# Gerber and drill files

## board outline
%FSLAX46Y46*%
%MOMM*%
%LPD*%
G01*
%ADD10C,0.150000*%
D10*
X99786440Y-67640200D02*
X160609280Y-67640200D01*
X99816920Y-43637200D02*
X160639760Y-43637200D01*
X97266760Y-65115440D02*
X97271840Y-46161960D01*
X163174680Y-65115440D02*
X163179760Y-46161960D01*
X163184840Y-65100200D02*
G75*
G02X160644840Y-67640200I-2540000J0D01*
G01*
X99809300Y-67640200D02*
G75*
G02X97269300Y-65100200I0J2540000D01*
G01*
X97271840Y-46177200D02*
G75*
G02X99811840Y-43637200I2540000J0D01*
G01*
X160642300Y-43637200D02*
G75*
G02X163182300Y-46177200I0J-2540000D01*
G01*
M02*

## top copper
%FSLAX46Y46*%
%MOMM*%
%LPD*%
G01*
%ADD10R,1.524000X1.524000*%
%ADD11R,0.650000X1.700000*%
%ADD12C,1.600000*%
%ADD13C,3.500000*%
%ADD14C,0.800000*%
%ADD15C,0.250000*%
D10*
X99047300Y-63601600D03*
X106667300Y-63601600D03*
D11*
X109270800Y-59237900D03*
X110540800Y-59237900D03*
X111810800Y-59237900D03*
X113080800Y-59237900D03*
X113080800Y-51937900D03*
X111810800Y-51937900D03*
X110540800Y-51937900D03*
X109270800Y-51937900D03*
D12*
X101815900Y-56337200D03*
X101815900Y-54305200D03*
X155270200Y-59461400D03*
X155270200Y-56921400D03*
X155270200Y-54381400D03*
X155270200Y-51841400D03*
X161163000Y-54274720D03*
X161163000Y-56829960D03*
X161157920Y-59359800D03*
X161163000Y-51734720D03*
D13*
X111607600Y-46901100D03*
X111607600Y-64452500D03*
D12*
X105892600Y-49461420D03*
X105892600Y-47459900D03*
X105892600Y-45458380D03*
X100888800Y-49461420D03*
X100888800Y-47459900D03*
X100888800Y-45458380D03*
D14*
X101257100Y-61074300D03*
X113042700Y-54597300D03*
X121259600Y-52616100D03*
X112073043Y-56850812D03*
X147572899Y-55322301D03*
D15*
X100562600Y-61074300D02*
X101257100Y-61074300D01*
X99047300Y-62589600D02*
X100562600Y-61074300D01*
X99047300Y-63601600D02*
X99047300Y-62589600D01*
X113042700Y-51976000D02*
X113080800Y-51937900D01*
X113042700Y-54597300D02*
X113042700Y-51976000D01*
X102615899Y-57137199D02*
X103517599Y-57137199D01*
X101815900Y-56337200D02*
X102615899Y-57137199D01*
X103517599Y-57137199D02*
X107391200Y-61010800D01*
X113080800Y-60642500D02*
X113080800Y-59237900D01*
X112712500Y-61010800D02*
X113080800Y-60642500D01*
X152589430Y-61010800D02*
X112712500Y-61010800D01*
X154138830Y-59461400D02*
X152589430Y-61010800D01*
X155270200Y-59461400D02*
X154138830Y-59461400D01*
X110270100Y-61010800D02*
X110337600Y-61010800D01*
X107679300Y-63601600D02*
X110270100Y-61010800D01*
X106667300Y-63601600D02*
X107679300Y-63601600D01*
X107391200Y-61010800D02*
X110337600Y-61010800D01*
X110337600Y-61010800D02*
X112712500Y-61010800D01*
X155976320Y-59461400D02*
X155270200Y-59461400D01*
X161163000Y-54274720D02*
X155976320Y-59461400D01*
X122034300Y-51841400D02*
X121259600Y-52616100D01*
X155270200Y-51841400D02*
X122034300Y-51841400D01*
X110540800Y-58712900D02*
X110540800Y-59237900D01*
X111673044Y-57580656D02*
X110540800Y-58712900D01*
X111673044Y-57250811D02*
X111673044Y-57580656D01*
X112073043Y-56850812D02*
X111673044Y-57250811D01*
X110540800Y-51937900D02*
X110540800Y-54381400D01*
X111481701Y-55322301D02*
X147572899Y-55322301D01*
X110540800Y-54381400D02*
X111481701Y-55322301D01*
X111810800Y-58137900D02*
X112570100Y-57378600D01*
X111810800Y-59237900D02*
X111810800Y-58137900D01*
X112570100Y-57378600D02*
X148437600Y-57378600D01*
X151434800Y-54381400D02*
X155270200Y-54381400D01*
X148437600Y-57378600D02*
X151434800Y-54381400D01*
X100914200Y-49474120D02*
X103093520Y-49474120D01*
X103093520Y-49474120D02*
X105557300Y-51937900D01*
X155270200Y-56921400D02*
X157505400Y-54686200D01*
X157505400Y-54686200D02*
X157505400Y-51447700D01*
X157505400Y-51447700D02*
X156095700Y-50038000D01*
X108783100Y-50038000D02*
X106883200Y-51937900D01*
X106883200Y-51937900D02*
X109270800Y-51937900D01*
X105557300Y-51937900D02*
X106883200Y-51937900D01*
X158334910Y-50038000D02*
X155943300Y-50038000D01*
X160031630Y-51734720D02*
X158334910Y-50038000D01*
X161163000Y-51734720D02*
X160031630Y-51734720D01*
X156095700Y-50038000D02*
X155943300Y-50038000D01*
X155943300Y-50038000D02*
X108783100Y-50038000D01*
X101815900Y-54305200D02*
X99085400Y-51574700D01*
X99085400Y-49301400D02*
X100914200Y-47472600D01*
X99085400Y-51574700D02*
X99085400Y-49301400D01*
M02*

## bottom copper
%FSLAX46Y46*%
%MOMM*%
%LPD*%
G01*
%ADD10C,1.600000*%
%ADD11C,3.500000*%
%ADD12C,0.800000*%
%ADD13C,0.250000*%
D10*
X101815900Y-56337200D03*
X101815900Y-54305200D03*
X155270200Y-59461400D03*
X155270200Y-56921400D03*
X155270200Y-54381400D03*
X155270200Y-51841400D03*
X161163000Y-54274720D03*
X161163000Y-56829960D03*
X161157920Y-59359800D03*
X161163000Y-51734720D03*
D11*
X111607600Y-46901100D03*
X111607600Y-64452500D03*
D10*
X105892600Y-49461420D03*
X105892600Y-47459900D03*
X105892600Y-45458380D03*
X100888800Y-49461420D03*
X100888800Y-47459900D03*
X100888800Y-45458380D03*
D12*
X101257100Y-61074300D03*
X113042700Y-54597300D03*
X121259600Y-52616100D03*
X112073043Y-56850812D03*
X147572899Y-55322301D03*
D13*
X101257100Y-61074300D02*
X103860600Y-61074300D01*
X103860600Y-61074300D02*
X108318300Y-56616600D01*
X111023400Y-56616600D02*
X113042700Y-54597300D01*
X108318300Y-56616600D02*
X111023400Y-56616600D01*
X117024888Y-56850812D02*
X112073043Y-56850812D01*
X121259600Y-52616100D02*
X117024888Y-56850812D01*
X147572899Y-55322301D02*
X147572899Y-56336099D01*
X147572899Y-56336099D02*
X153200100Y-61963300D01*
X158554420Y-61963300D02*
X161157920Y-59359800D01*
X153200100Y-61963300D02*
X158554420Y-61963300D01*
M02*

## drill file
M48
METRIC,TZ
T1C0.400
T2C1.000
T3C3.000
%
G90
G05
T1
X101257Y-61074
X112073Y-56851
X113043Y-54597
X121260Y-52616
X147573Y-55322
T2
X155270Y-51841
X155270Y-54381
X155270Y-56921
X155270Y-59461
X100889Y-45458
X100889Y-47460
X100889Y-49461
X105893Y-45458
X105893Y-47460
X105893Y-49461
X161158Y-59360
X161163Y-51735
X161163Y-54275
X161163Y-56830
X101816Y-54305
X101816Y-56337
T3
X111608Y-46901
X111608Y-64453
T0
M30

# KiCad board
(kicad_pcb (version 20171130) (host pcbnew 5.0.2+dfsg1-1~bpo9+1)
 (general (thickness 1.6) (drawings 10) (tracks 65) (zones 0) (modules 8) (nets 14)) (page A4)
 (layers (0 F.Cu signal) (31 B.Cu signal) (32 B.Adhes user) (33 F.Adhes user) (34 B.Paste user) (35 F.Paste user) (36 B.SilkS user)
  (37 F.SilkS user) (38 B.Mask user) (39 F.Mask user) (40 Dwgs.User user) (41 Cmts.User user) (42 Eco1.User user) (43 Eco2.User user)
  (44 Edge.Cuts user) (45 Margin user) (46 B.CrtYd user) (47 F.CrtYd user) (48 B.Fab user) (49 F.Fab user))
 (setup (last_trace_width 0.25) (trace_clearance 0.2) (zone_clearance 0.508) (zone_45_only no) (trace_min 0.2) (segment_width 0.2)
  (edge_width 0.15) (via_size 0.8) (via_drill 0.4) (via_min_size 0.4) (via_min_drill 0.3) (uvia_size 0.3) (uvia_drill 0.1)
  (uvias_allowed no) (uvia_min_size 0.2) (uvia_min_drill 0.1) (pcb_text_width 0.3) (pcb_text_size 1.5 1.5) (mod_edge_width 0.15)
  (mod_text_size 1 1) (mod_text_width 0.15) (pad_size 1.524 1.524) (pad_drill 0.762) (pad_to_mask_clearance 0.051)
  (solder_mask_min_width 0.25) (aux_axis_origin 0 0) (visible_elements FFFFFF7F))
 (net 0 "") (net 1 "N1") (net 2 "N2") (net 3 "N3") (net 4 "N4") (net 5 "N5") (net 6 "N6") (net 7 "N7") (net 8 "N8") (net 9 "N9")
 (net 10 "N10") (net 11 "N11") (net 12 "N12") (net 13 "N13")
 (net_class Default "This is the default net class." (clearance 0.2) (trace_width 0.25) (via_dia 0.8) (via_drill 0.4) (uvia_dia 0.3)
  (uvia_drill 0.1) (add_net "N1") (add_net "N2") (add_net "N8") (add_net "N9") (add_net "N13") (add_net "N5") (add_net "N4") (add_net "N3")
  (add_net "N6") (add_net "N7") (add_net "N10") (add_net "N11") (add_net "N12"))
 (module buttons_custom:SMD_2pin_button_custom (layer F.Cu) (at 102.8573 63.6016 180)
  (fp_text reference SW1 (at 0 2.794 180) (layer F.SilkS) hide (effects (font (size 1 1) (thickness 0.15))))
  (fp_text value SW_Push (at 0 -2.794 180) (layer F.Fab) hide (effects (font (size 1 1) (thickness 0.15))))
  (pad 1 smd rect (at 3.81 0 180) (size 1.524 1.524) (layers F.Cu F.Paste F.Mask) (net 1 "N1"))
  (pad 2 smd rect (at -3.81 0 180) (size 1.524 1.524) (layers F.Cu F.Paste F.Mask) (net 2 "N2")))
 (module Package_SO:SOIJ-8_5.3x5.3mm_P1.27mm (layer F.Cu) (at 111.1758 55.5879 90)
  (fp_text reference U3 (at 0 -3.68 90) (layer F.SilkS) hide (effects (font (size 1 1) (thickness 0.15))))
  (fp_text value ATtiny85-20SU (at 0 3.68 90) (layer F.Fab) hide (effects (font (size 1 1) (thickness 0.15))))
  (pad 1 smd rect (at -3.65 -1.905 90) (size 1.7 0.65) (layers F.Cu F.Paste F.Mask) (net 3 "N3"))
  (pad 2 smd rect (at -3.65 -0.635 90) (size 1.7 0.65) (layers F.Cu F.Paste F.Mask) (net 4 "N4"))
  (pad 3 smd rect (at -3.65 0.635 90) (size 1.7 0.65) (layers F.Cu F.Paste F.Mask) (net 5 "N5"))
  (pad 4 smd rect (at -3.65 1.905 90) (size 1.7 0.65) (layers F.Cu F.Paste F.Mask) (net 2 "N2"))
  (pad 5 smd rect (at 3.65 1.905 90) (size 1.7 0.65) (layers F.Cu F.Paste F.Mask) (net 1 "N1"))
  (pad 6 smd rect (at 3.65 0.635 90) (size 1.7 0.65) (layers F.Cu F.Paste F.Mask) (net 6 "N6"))
  (pad 7 smd rect (at 3.65 -0.635 90) (size 1.7 0.65) (layers F.Cu F.Paste F.Mask) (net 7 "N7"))
  (pad 8 smd rect (at 3.65 -1.905 90) (size 1.7 0.65) (layers F.Cu F.Paste F.Mask) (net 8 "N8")))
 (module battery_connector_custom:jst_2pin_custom (layer F.Cu) (at 101.8159 55.3212 90)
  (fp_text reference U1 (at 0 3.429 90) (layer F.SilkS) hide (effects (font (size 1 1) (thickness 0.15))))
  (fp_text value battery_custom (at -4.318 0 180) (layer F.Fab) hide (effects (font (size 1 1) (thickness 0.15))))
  (pad 1 thru_hole circle (at -1.016 0 90) (size 1.6 1.6) (drill 1) (layers *.Cu *.Mask) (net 2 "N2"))
  (pad 2 thru_hole circle (at 1.016 0 90) (size 1.6 1.6) (drill 1) (layers *.Cu *.Mask) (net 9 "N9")))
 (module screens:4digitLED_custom (layer F.Cu) (at 155.2702 55.6514 90)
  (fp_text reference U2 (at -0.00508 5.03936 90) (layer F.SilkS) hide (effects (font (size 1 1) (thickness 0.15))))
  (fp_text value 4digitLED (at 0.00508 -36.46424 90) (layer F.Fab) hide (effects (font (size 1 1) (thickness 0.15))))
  (pad 1 thru_hole circle (at -3.81 0 90) (size 1.6 1.6) (drill 1) (layers *.Cu *.Mask) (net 2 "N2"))
  (pad 2 thru_hole circle (at -1.27 0 90) (size 1.6 1.6) (drill 1) (layers *.Cu *.Mask) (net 8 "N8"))
  (pad 3 thru_hole circle (at 1.27 0 90) (size 1.6 1.6) (drill 1) (layers *.Cu *.Mask) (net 5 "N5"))
  (pad 4 thru_hole circle (at 3.81 0 90) (size 1.6 1.6) (drill 1) (layers *.Cu *.Mask) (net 4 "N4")))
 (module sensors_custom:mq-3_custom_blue (layer F.Cu) (at 161.163 55.5498 270)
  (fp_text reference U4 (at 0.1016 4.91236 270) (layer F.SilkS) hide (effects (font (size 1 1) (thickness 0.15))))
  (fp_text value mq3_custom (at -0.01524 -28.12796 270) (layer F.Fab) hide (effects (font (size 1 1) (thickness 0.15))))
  (pad 2 thru_hole circle (at -1.27508 0 270) (size 1.6 1.6) (drill 1) (layers *.Cu *.Mask) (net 2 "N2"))
  (pad 3 thru_hole circle (at 1.28016 0 270) (size 1.6 1.6) (drill 1) (layers *.Cu *.Mask) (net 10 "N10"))
  (pad 4 thru_hole circle (at 3.81 0.00508 270) (size 1.6 1.6) (drill 1) (layers *.Cu *.Mask) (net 7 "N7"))
  (pad 1 thru_hole circle (at -3.81508 0 270) (size 1.6 1.6) (drill 1) (layers *.Cu *.Mask) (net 8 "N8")))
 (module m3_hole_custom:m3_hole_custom (layer F.Cu) (at 111.6076 46.9011)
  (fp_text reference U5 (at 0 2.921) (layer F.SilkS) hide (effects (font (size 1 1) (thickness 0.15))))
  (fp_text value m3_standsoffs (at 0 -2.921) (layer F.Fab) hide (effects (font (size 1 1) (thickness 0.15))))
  (pad 1 thru_hole circle (at 0 0) (size 3.5 3.5) (drill 3) (layers *.Cu *.Mask) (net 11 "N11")))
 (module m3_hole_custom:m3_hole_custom (layer F.Cu) (at 111.6076 64.4525)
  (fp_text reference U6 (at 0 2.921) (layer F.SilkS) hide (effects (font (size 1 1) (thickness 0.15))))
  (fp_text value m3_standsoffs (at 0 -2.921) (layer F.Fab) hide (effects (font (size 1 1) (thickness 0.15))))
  (pad 1 thru_hole circle (at 0 0) (size 3.5 3.5) (drill 3) (layers *.Cu *.Mask) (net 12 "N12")))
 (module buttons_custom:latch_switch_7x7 (layer F.Cu) (at 105.8926 47.4599 90)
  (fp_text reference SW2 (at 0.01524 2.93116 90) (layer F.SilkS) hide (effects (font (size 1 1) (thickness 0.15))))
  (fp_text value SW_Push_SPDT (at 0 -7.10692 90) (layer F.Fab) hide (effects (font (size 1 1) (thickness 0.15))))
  (pad 4 thru_hole circle (at -2.00152 0 90) (size 1.6 1.6) (drill 1) (layers *.Cu *.Mask))
  (pad 5 thru_hole circle (at 0 0 90) (size 1.6 1.6) (drill 1) (layers *.Cu *.Mask))
  (pad 6 thru_hole circle (at 2.00152 0 90) (size 1.6 1.6) (drill 1) (layers *.Cu *.Mask))
  (pad 1 thru_hole circle (at -2.00152 -5.0038 90) (size 1.6 1.6) (drill 1) (layers *.Cu *.Mask) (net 8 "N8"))
  (pad 2 thru_hole circle (at 0 -5.0038 90) (size 1.6 1.6) (drill 1) (layers *.Cu *.Mask) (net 9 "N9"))
  (pad 3 thru_hole circle (at 2.00152 -5.0038 90) (size 1.6 1.6) (drill 1) (layers *.Cu *.Mask) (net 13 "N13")))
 (gr_line (start 99.78644 67.6402) (end 160.60928 67.6402) (layer Edge.Cuts) (width 0.15))
 (gr_line (start 99.81692 43.6372) (end 160.63976 43.6372) (layer Edge.Cuts) (width 0.15))
 (gr_line (start 97.26676 65.11544) (end 97.27184 46.16196) (layer Edge.Cuts) (width 0.15))
 (gr_line (start 163.17468 65.11544) (end 163.17976 46.16196) (layer Edge.Cuts) (width 0.15))
 (gr_arc (start 160.64484 65.1002) (end 160.64484 67.6402) (angle -90) (layer Edge.Cuts) (width 0.15))
 (gr_arc (start 99.8093 65.1002) (end 97.2693 65.1002) (angle -90) (layer Edge.Cuts) (width 0.15))
 (gr_arc (start 99.81184 46.1772) (end 99.81184 43.6372) (angle -90) (layer Edge.Cuts) (width 0.15))
 (gr_arc (start 160.6423 46.1772) (end 163.1823 46.1772) (angle -90) (layer Edge.Cuts) (width 0.15))
 (via (at 101.2571 61.0743) (size 0.8) (drill 0.4) (layers F.Cu B.Cu) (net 1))
 (segment (start 100.5626 61.0743) (end 101.2571 61.0743) (width 0.25) (layer F.Cu) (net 1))
 (segment (start 99.0473 62.5896) (end 100.5626 61.0743) (width 0.25) (layer F.Cu) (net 1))
 (segment (start 99.0473 63.6016) (end 99.0473 62.5896) (width 0.25) (layer F.Cu) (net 1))
 (segment (start 101.2571 61.0743) (end 103.8606 61.0743) (width 0.25) (layer B.Cu) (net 1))
 (segment (start 103.8606 61.0743) (end 108.3183 56.6166) (width 0.25) (layer B.Cu) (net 1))
 (segment (start 111.0234 56.6166) (end 113.0427 54.5973) (width 0.25) (layer B.Cu) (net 1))
 (via (at 113.0427 54.5973) (size 0.8) (drill 0.4) (layers F.Cu B.Cu) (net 1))
 (segment (start 108.3183 56.6166) (end 111.0234 56.6166) (width 0.25) (layer B.Cu) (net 1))
 (segment (start 113.0427 51.976) (end 113.0808 51.9379) (width 0.25) (layer F.Cu) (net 1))
 (segment (start 113.0427 54.5973) (end 113.0427 51.976) (width 0.25) (layer F.Cu) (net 1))
 (segment (start 102.615899 57.137199) (end 103.517599 57.137199) (width 0.25) (layer F.Cu) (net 2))
 (segment (start 101.8159 56.3372) (end 102.615899 57.137199) (width 0.25) (layer F.Cu) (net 2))
 (segment (start 103.517599 57.137199) (end 107.3912 61.0108) (width 0.25) (layer F.Cu) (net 2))
 (segment (start 113.0808 60.6425) (end 113.0808 59.2379) (width 0.25) (layer F.Cu) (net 2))
 (segment (start 112.7125 61.0108) (end 113.0808 60.6425) (width 0.25) (layer F.Cu) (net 2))
 (segment (start 152.58943 61.0108) (end 112.7125 61.0108) (width 0.25) (layer F.Cu) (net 2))
 (segment (start 154.13883 59.4614) (end 152.58943 61.0108) (width 0.25) (layer F.Cu) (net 2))
 (segment (start 155.2702 59.4614) (end 154.13883 59.4614) (width 0.25) (layer F.Cu) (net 2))
 (segment (start 110.2701 61.0108) (end 110.3376 61.0108) (width 0.25) (layer F.Cu) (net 2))
 (segment (start 107.6793 63.6016) (end 110.2701 61.0108) (width 0.25) (layer F.Cu) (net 2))
 (segment (start 106.6673 63.6016) (end 107.6793 63.6016) (width 0.25) (layer F.Cu) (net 2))
 (segment (start 107.3912 61.0108) (end 110.3376 61.0108) (width 0.25) (layer F.Cu) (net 2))
 (segment (start 110.3376 61.0108) (end 112.7125 61.0108) (width 0.25) (layer F.Cu) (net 2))
 (segment (start 155.97632 59.4614) (end 155.2702 59.4614) (width 0.25) (layer F.Cu) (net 2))
 (segment (start 161.163 54.27472) (end 155.97632 59.4614) (width 0.25) (layer F.Cu) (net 2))
 (via (at 121.2596 52.6161) (size 0.8) (drill 0.4) (layers F.Cu B.Cu) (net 4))
 (segment (start 122.0343 51.8414) (end 121.2596 52.6161) (width 0.25) (layer F.Cu) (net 4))
 (segment (start 155.2702 51.8414) (end 122.0343 51.8414) (width 0.25) (layer F.Cu) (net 4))
 (via (at 112.073043 56.850812) (size 0.8) (drill 0.4) (layers F.Cu B.Cu) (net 4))
 (segment (start 117.024888 56.850812) (end 112.073043 56.850812) (width 0.25) (layer B.Cu) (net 4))
 (segment (start 121.2596 52.6161) (end 117.024888 56.850812) (width 0.25) (layer B.Cu) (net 4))
 (segment (start 110.5408 58.7129) (end 110.5408 59.2379) (width 0.25) (layer F.Cu) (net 4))
 (segment (start 111.673044 57.580656) (end 110.5408 58.7129) (width 0.25) (layer F.Cu) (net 4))
 (segment (start 111.673044 57.250811) (end 111.673044 57.580656) (width 0.25) (layer F.Cu) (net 4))
 (segment (start 112.073043 56.850812) (end 111.673044 57.250811) (width 0.25) (layer F.Cu) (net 4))
 (segment (start 110.5408 51.9379) (end 110.5408 54.3814) (width 0.25) (layer F.Cu) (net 7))
 (segment (start 111.481701 55.322301) (end 147.572899 55.322301) (width 0.25) (layer F.Cu) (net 7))
 (segment (start 110.5408 54.3814) (end 111.481701 55.322301) (width 0.25) (layer F.Cu) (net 7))
 (via (at 147.572899 55.322301) (size 0.8) (drill 0.4) (layers F.Cu B.Cu) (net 7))
 (segment (start 147.572899 55.322301) (end 147.572899 56.336099) (width 0.25) (layer B.Cu) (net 7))
 (segment (start 147.572899 56.336099) (end 153.2001 61.9633) (width 0.25) (layer B.Cu) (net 7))
 (segment (start 158.55442 61.9633) (end 161.15792 59.3598) (width 0.25) (layer B.Cu) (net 7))
 (segment (start 153.2001 61.9633) (end 158.55442 61.9633) (width 0.25) (layer B.Cu) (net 7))
 (segment (start 111.8108 58.1379) (end 112.5701 57.3786) (width 0.25) (layer F.Cu) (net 5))
 (segment (start 111.8108 59.2379) (end 111.8108 58.1379) (width 0.25) (layer F.Cu) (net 5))
 (segment (start 112.5701 57.3786) (end 148.4376 57.3786) (width 0.25) (layer F.Cu) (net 5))
 (segment (start 151.4348 54.3814) (end 155.2702 54.3814) (width 0.25) (layer F.Cu) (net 5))
 (segment (start 148.4376 57.3786) (end 151.4348 54.3814) (width 0.25) (layer F.Cu) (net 5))
 (segment (start 100.9142 49.47412) (end 103.09352 49.47412) (width 0.25) (layer F.Cu) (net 8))
 (segment (start 103.09352 49.47412) (end 105.5573 51.9379) (width 0.25) (layer F.Cu) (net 8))
 (segment (start 155.2702 56.9214) (end 157.5054 54.6862) (width 0.25) (layer F.Cu) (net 8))
 (segment (start 157.5054 54.6862) (end 157.5054 51.4477) (width 0.25) (layer F.Cu) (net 8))
 (segment (start 157.5054 51.4477) (end 156.0957 50.038) (width 0.25) (layer F.Cu) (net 8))
 (segment (start 108.7831 50.038) (end 106.8832 51.9379) (width 0.25) (layer F.Cu) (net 8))
 (segment (start 106.8832 51.9379) (end 109.2708 51.9379) (width 0.25) (layer F.Cu) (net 8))
 (segment (start 105.5573 51.9379) (end 106.8832 51.9379) (width 0.25) (layer F.Cu) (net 8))
 (segment (start 158.33491 50.038) (end 155.9433 50.038) (width 0.25) (layer F.Cu) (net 8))
 (segment (start 160.03163 51.73472) (end 158.33491 50.038) (width 0.25) (layer F.Cu) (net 8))
 (segment (start 161.163 51.73472) (end 160.03163 51.73472) (width 0.25) (layer F.Cu) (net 8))
 (segment (start 156.0957 50.038) (end 155.9433 50.038) (width 0.25) (layer F.Cu) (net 8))
 (segment (start 155.9433 50.038) (end 108.7831 50.038) (width 0.25) (layer F.Cu) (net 8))
 (segment (start 101.8159 54.3052) (end 99.0854 51.5747) (width 0.25) (layer F.Cu) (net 9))
 (segment (start 99.0854 49.3014) (end 100.9142 47.4726) (width 0.25) (layer F.Cu) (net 9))
 (segment (start 99.0854 51.5747) (end 99.0854 49.3014) (width 0.25) (layer F.Cu) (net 9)))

